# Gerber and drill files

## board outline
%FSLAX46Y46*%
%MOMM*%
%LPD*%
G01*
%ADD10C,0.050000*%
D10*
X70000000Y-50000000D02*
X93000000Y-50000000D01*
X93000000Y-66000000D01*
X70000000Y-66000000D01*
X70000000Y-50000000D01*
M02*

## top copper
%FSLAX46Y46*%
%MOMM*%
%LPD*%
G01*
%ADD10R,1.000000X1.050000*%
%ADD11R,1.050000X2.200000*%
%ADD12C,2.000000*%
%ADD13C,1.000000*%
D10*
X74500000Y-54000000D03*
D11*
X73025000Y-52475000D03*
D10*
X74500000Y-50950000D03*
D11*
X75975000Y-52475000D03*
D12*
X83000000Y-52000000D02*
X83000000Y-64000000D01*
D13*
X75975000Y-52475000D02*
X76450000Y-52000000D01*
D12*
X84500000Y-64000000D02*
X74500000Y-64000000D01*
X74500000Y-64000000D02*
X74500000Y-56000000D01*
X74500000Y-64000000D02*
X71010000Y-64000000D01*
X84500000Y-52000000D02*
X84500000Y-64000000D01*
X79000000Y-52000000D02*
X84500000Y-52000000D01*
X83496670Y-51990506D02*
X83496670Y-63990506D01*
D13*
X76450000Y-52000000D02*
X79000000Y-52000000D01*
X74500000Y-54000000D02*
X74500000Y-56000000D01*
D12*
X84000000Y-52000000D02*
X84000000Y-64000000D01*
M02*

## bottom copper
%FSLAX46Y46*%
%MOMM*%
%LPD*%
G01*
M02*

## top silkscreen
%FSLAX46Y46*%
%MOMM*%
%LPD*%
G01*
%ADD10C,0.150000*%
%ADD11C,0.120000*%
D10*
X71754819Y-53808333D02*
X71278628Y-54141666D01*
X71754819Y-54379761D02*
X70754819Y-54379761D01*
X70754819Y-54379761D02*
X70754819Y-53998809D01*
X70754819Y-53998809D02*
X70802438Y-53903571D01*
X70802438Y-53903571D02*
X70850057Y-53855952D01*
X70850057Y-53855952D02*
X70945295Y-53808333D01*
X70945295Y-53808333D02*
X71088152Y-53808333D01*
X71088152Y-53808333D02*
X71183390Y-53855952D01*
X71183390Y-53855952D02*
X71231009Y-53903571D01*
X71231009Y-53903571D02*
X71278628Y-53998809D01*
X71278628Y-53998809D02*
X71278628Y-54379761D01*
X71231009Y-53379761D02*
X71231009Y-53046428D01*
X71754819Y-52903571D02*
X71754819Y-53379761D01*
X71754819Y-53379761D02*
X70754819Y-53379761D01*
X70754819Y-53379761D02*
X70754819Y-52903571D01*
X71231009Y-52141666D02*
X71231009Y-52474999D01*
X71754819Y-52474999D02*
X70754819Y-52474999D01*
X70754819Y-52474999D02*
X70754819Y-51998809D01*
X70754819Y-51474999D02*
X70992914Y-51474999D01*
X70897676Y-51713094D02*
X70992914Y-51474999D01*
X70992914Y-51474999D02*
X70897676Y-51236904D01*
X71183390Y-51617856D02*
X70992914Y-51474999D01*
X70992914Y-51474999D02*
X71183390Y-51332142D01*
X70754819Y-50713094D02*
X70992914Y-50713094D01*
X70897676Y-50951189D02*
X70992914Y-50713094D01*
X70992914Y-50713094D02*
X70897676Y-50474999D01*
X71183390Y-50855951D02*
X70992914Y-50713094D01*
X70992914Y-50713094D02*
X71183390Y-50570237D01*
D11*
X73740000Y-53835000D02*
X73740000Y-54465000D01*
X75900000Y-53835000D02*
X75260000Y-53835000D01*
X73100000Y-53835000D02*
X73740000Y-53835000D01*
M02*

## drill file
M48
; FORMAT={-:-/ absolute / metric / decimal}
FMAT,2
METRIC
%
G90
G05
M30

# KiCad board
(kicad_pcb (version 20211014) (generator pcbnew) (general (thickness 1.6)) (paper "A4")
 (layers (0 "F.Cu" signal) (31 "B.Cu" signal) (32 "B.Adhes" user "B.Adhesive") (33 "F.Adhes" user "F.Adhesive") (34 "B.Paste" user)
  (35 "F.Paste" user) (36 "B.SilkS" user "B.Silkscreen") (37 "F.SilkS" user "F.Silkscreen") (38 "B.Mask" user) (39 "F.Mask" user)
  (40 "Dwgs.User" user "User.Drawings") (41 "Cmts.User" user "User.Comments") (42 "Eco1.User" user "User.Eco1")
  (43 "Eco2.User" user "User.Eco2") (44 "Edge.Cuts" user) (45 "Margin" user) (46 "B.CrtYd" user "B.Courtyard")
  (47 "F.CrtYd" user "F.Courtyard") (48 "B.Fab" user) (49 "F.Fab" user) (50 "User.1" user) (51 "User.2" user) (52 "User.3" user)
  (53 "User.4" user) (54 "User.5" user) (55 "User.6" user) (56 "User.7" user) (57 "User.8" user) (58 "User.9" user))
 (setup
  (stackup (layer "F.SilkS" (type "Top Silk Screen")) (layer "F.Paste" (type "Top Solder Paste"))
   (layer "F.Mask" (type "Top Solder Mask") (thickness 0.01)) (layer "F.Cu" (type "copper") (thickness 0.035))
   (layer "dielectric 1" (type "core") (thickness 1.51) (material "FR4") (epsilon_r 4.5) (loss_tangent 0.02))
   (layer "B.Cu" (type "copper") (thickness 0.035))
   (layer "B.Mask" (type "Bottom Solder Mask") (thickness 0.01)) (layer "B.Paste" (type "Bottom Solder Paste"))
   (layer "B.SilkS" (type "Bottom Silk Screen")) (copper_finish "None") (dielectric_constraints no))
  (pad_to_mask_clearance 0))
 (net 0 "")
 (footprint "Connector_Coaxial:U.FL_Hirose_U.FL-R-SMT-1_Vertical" (layer "F.Cu") (at 74.5 52.95 90)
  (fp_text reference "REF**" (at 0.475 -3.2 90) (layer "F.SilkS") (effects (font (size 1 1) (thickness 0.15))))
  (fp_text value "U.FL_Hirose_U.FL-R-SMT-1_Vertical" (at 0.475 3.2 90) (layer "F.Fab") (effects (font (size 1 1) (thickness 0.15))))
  (fp_line (start -0.885 -0.76) (end -1.515 -0.76) (layer "F.SilkS") (width 0.12))
  (fp_line (start -0.885 1.4) (end -0.885 0.76) (layer "F.SilkS") (width 0.12))
  (fp_line (start -0.885 -1.4) (end -0.885 -0.76) (layer "F.SilkS") (width 0.12))
  (pad "1" smd rect (at -1.05 0 90) (size 1.05 1) (layers "F.Cu" "F.Paste" "F.Mask"))
  (pad "2" smd rect (at 0.475 -1.475 90) (size 2.2 1.05) (layers "F.Cu" "F.Paste" "F.Mask"))
  (pad "2" smd rect (at 2 0 90) (size 1.05 1) (layers "F.Cu" "F.Paste" "F.Mask"))
  (pad "2" smd rect (at 0.475 1.475 90) (size 2.2 1.05) (layers "F.Cu" "F.Paste" "F.Mask")))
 (gr_rect (start 70 50) (end 93 66) (layer "Edge.Cuts") (width 0.05) (fill none))
 (segment (start 83 52) (end 83 64) (width 2) (layer "F.Cu") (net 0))
 (segment (start 75.975 52.475) (end 76.45 52) (width 1) (layer "F.Cu") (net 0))
 (segment (start 84.5 64) (end 74.5 64) (width 2) (layer "F.Cu") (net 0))
 (segment (start 74.5 64) (end 74.5 56) (width 2) (layer "F.Cu") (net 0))
 (segment (start 74.5 64) (end 71.01 64) (width 2) (layer "F.Cu") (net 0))
 (segment (start 84.5 52) (end 84.5 64) (width 2) (layer "F.Cu") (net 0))
 (segment (start 79 52) (end 84.5 52) (width 2) (layer "F.Cu") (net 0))
 (segment (start 83.49667 51.990506) (end 83.49667 63.990506) (width 2) (layer "F.Cu") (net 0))
 (segment (start 76.45 52) (end 79 52) (width 1) (layer "F.Cu") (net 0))
 (segment (start 74.5 54) (end 74.5 56) (width 1) (layer "F.Cu") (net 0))
 (segment (start 84 52) (end 84 64) (width 2) (layer "F.Cu") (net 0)))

